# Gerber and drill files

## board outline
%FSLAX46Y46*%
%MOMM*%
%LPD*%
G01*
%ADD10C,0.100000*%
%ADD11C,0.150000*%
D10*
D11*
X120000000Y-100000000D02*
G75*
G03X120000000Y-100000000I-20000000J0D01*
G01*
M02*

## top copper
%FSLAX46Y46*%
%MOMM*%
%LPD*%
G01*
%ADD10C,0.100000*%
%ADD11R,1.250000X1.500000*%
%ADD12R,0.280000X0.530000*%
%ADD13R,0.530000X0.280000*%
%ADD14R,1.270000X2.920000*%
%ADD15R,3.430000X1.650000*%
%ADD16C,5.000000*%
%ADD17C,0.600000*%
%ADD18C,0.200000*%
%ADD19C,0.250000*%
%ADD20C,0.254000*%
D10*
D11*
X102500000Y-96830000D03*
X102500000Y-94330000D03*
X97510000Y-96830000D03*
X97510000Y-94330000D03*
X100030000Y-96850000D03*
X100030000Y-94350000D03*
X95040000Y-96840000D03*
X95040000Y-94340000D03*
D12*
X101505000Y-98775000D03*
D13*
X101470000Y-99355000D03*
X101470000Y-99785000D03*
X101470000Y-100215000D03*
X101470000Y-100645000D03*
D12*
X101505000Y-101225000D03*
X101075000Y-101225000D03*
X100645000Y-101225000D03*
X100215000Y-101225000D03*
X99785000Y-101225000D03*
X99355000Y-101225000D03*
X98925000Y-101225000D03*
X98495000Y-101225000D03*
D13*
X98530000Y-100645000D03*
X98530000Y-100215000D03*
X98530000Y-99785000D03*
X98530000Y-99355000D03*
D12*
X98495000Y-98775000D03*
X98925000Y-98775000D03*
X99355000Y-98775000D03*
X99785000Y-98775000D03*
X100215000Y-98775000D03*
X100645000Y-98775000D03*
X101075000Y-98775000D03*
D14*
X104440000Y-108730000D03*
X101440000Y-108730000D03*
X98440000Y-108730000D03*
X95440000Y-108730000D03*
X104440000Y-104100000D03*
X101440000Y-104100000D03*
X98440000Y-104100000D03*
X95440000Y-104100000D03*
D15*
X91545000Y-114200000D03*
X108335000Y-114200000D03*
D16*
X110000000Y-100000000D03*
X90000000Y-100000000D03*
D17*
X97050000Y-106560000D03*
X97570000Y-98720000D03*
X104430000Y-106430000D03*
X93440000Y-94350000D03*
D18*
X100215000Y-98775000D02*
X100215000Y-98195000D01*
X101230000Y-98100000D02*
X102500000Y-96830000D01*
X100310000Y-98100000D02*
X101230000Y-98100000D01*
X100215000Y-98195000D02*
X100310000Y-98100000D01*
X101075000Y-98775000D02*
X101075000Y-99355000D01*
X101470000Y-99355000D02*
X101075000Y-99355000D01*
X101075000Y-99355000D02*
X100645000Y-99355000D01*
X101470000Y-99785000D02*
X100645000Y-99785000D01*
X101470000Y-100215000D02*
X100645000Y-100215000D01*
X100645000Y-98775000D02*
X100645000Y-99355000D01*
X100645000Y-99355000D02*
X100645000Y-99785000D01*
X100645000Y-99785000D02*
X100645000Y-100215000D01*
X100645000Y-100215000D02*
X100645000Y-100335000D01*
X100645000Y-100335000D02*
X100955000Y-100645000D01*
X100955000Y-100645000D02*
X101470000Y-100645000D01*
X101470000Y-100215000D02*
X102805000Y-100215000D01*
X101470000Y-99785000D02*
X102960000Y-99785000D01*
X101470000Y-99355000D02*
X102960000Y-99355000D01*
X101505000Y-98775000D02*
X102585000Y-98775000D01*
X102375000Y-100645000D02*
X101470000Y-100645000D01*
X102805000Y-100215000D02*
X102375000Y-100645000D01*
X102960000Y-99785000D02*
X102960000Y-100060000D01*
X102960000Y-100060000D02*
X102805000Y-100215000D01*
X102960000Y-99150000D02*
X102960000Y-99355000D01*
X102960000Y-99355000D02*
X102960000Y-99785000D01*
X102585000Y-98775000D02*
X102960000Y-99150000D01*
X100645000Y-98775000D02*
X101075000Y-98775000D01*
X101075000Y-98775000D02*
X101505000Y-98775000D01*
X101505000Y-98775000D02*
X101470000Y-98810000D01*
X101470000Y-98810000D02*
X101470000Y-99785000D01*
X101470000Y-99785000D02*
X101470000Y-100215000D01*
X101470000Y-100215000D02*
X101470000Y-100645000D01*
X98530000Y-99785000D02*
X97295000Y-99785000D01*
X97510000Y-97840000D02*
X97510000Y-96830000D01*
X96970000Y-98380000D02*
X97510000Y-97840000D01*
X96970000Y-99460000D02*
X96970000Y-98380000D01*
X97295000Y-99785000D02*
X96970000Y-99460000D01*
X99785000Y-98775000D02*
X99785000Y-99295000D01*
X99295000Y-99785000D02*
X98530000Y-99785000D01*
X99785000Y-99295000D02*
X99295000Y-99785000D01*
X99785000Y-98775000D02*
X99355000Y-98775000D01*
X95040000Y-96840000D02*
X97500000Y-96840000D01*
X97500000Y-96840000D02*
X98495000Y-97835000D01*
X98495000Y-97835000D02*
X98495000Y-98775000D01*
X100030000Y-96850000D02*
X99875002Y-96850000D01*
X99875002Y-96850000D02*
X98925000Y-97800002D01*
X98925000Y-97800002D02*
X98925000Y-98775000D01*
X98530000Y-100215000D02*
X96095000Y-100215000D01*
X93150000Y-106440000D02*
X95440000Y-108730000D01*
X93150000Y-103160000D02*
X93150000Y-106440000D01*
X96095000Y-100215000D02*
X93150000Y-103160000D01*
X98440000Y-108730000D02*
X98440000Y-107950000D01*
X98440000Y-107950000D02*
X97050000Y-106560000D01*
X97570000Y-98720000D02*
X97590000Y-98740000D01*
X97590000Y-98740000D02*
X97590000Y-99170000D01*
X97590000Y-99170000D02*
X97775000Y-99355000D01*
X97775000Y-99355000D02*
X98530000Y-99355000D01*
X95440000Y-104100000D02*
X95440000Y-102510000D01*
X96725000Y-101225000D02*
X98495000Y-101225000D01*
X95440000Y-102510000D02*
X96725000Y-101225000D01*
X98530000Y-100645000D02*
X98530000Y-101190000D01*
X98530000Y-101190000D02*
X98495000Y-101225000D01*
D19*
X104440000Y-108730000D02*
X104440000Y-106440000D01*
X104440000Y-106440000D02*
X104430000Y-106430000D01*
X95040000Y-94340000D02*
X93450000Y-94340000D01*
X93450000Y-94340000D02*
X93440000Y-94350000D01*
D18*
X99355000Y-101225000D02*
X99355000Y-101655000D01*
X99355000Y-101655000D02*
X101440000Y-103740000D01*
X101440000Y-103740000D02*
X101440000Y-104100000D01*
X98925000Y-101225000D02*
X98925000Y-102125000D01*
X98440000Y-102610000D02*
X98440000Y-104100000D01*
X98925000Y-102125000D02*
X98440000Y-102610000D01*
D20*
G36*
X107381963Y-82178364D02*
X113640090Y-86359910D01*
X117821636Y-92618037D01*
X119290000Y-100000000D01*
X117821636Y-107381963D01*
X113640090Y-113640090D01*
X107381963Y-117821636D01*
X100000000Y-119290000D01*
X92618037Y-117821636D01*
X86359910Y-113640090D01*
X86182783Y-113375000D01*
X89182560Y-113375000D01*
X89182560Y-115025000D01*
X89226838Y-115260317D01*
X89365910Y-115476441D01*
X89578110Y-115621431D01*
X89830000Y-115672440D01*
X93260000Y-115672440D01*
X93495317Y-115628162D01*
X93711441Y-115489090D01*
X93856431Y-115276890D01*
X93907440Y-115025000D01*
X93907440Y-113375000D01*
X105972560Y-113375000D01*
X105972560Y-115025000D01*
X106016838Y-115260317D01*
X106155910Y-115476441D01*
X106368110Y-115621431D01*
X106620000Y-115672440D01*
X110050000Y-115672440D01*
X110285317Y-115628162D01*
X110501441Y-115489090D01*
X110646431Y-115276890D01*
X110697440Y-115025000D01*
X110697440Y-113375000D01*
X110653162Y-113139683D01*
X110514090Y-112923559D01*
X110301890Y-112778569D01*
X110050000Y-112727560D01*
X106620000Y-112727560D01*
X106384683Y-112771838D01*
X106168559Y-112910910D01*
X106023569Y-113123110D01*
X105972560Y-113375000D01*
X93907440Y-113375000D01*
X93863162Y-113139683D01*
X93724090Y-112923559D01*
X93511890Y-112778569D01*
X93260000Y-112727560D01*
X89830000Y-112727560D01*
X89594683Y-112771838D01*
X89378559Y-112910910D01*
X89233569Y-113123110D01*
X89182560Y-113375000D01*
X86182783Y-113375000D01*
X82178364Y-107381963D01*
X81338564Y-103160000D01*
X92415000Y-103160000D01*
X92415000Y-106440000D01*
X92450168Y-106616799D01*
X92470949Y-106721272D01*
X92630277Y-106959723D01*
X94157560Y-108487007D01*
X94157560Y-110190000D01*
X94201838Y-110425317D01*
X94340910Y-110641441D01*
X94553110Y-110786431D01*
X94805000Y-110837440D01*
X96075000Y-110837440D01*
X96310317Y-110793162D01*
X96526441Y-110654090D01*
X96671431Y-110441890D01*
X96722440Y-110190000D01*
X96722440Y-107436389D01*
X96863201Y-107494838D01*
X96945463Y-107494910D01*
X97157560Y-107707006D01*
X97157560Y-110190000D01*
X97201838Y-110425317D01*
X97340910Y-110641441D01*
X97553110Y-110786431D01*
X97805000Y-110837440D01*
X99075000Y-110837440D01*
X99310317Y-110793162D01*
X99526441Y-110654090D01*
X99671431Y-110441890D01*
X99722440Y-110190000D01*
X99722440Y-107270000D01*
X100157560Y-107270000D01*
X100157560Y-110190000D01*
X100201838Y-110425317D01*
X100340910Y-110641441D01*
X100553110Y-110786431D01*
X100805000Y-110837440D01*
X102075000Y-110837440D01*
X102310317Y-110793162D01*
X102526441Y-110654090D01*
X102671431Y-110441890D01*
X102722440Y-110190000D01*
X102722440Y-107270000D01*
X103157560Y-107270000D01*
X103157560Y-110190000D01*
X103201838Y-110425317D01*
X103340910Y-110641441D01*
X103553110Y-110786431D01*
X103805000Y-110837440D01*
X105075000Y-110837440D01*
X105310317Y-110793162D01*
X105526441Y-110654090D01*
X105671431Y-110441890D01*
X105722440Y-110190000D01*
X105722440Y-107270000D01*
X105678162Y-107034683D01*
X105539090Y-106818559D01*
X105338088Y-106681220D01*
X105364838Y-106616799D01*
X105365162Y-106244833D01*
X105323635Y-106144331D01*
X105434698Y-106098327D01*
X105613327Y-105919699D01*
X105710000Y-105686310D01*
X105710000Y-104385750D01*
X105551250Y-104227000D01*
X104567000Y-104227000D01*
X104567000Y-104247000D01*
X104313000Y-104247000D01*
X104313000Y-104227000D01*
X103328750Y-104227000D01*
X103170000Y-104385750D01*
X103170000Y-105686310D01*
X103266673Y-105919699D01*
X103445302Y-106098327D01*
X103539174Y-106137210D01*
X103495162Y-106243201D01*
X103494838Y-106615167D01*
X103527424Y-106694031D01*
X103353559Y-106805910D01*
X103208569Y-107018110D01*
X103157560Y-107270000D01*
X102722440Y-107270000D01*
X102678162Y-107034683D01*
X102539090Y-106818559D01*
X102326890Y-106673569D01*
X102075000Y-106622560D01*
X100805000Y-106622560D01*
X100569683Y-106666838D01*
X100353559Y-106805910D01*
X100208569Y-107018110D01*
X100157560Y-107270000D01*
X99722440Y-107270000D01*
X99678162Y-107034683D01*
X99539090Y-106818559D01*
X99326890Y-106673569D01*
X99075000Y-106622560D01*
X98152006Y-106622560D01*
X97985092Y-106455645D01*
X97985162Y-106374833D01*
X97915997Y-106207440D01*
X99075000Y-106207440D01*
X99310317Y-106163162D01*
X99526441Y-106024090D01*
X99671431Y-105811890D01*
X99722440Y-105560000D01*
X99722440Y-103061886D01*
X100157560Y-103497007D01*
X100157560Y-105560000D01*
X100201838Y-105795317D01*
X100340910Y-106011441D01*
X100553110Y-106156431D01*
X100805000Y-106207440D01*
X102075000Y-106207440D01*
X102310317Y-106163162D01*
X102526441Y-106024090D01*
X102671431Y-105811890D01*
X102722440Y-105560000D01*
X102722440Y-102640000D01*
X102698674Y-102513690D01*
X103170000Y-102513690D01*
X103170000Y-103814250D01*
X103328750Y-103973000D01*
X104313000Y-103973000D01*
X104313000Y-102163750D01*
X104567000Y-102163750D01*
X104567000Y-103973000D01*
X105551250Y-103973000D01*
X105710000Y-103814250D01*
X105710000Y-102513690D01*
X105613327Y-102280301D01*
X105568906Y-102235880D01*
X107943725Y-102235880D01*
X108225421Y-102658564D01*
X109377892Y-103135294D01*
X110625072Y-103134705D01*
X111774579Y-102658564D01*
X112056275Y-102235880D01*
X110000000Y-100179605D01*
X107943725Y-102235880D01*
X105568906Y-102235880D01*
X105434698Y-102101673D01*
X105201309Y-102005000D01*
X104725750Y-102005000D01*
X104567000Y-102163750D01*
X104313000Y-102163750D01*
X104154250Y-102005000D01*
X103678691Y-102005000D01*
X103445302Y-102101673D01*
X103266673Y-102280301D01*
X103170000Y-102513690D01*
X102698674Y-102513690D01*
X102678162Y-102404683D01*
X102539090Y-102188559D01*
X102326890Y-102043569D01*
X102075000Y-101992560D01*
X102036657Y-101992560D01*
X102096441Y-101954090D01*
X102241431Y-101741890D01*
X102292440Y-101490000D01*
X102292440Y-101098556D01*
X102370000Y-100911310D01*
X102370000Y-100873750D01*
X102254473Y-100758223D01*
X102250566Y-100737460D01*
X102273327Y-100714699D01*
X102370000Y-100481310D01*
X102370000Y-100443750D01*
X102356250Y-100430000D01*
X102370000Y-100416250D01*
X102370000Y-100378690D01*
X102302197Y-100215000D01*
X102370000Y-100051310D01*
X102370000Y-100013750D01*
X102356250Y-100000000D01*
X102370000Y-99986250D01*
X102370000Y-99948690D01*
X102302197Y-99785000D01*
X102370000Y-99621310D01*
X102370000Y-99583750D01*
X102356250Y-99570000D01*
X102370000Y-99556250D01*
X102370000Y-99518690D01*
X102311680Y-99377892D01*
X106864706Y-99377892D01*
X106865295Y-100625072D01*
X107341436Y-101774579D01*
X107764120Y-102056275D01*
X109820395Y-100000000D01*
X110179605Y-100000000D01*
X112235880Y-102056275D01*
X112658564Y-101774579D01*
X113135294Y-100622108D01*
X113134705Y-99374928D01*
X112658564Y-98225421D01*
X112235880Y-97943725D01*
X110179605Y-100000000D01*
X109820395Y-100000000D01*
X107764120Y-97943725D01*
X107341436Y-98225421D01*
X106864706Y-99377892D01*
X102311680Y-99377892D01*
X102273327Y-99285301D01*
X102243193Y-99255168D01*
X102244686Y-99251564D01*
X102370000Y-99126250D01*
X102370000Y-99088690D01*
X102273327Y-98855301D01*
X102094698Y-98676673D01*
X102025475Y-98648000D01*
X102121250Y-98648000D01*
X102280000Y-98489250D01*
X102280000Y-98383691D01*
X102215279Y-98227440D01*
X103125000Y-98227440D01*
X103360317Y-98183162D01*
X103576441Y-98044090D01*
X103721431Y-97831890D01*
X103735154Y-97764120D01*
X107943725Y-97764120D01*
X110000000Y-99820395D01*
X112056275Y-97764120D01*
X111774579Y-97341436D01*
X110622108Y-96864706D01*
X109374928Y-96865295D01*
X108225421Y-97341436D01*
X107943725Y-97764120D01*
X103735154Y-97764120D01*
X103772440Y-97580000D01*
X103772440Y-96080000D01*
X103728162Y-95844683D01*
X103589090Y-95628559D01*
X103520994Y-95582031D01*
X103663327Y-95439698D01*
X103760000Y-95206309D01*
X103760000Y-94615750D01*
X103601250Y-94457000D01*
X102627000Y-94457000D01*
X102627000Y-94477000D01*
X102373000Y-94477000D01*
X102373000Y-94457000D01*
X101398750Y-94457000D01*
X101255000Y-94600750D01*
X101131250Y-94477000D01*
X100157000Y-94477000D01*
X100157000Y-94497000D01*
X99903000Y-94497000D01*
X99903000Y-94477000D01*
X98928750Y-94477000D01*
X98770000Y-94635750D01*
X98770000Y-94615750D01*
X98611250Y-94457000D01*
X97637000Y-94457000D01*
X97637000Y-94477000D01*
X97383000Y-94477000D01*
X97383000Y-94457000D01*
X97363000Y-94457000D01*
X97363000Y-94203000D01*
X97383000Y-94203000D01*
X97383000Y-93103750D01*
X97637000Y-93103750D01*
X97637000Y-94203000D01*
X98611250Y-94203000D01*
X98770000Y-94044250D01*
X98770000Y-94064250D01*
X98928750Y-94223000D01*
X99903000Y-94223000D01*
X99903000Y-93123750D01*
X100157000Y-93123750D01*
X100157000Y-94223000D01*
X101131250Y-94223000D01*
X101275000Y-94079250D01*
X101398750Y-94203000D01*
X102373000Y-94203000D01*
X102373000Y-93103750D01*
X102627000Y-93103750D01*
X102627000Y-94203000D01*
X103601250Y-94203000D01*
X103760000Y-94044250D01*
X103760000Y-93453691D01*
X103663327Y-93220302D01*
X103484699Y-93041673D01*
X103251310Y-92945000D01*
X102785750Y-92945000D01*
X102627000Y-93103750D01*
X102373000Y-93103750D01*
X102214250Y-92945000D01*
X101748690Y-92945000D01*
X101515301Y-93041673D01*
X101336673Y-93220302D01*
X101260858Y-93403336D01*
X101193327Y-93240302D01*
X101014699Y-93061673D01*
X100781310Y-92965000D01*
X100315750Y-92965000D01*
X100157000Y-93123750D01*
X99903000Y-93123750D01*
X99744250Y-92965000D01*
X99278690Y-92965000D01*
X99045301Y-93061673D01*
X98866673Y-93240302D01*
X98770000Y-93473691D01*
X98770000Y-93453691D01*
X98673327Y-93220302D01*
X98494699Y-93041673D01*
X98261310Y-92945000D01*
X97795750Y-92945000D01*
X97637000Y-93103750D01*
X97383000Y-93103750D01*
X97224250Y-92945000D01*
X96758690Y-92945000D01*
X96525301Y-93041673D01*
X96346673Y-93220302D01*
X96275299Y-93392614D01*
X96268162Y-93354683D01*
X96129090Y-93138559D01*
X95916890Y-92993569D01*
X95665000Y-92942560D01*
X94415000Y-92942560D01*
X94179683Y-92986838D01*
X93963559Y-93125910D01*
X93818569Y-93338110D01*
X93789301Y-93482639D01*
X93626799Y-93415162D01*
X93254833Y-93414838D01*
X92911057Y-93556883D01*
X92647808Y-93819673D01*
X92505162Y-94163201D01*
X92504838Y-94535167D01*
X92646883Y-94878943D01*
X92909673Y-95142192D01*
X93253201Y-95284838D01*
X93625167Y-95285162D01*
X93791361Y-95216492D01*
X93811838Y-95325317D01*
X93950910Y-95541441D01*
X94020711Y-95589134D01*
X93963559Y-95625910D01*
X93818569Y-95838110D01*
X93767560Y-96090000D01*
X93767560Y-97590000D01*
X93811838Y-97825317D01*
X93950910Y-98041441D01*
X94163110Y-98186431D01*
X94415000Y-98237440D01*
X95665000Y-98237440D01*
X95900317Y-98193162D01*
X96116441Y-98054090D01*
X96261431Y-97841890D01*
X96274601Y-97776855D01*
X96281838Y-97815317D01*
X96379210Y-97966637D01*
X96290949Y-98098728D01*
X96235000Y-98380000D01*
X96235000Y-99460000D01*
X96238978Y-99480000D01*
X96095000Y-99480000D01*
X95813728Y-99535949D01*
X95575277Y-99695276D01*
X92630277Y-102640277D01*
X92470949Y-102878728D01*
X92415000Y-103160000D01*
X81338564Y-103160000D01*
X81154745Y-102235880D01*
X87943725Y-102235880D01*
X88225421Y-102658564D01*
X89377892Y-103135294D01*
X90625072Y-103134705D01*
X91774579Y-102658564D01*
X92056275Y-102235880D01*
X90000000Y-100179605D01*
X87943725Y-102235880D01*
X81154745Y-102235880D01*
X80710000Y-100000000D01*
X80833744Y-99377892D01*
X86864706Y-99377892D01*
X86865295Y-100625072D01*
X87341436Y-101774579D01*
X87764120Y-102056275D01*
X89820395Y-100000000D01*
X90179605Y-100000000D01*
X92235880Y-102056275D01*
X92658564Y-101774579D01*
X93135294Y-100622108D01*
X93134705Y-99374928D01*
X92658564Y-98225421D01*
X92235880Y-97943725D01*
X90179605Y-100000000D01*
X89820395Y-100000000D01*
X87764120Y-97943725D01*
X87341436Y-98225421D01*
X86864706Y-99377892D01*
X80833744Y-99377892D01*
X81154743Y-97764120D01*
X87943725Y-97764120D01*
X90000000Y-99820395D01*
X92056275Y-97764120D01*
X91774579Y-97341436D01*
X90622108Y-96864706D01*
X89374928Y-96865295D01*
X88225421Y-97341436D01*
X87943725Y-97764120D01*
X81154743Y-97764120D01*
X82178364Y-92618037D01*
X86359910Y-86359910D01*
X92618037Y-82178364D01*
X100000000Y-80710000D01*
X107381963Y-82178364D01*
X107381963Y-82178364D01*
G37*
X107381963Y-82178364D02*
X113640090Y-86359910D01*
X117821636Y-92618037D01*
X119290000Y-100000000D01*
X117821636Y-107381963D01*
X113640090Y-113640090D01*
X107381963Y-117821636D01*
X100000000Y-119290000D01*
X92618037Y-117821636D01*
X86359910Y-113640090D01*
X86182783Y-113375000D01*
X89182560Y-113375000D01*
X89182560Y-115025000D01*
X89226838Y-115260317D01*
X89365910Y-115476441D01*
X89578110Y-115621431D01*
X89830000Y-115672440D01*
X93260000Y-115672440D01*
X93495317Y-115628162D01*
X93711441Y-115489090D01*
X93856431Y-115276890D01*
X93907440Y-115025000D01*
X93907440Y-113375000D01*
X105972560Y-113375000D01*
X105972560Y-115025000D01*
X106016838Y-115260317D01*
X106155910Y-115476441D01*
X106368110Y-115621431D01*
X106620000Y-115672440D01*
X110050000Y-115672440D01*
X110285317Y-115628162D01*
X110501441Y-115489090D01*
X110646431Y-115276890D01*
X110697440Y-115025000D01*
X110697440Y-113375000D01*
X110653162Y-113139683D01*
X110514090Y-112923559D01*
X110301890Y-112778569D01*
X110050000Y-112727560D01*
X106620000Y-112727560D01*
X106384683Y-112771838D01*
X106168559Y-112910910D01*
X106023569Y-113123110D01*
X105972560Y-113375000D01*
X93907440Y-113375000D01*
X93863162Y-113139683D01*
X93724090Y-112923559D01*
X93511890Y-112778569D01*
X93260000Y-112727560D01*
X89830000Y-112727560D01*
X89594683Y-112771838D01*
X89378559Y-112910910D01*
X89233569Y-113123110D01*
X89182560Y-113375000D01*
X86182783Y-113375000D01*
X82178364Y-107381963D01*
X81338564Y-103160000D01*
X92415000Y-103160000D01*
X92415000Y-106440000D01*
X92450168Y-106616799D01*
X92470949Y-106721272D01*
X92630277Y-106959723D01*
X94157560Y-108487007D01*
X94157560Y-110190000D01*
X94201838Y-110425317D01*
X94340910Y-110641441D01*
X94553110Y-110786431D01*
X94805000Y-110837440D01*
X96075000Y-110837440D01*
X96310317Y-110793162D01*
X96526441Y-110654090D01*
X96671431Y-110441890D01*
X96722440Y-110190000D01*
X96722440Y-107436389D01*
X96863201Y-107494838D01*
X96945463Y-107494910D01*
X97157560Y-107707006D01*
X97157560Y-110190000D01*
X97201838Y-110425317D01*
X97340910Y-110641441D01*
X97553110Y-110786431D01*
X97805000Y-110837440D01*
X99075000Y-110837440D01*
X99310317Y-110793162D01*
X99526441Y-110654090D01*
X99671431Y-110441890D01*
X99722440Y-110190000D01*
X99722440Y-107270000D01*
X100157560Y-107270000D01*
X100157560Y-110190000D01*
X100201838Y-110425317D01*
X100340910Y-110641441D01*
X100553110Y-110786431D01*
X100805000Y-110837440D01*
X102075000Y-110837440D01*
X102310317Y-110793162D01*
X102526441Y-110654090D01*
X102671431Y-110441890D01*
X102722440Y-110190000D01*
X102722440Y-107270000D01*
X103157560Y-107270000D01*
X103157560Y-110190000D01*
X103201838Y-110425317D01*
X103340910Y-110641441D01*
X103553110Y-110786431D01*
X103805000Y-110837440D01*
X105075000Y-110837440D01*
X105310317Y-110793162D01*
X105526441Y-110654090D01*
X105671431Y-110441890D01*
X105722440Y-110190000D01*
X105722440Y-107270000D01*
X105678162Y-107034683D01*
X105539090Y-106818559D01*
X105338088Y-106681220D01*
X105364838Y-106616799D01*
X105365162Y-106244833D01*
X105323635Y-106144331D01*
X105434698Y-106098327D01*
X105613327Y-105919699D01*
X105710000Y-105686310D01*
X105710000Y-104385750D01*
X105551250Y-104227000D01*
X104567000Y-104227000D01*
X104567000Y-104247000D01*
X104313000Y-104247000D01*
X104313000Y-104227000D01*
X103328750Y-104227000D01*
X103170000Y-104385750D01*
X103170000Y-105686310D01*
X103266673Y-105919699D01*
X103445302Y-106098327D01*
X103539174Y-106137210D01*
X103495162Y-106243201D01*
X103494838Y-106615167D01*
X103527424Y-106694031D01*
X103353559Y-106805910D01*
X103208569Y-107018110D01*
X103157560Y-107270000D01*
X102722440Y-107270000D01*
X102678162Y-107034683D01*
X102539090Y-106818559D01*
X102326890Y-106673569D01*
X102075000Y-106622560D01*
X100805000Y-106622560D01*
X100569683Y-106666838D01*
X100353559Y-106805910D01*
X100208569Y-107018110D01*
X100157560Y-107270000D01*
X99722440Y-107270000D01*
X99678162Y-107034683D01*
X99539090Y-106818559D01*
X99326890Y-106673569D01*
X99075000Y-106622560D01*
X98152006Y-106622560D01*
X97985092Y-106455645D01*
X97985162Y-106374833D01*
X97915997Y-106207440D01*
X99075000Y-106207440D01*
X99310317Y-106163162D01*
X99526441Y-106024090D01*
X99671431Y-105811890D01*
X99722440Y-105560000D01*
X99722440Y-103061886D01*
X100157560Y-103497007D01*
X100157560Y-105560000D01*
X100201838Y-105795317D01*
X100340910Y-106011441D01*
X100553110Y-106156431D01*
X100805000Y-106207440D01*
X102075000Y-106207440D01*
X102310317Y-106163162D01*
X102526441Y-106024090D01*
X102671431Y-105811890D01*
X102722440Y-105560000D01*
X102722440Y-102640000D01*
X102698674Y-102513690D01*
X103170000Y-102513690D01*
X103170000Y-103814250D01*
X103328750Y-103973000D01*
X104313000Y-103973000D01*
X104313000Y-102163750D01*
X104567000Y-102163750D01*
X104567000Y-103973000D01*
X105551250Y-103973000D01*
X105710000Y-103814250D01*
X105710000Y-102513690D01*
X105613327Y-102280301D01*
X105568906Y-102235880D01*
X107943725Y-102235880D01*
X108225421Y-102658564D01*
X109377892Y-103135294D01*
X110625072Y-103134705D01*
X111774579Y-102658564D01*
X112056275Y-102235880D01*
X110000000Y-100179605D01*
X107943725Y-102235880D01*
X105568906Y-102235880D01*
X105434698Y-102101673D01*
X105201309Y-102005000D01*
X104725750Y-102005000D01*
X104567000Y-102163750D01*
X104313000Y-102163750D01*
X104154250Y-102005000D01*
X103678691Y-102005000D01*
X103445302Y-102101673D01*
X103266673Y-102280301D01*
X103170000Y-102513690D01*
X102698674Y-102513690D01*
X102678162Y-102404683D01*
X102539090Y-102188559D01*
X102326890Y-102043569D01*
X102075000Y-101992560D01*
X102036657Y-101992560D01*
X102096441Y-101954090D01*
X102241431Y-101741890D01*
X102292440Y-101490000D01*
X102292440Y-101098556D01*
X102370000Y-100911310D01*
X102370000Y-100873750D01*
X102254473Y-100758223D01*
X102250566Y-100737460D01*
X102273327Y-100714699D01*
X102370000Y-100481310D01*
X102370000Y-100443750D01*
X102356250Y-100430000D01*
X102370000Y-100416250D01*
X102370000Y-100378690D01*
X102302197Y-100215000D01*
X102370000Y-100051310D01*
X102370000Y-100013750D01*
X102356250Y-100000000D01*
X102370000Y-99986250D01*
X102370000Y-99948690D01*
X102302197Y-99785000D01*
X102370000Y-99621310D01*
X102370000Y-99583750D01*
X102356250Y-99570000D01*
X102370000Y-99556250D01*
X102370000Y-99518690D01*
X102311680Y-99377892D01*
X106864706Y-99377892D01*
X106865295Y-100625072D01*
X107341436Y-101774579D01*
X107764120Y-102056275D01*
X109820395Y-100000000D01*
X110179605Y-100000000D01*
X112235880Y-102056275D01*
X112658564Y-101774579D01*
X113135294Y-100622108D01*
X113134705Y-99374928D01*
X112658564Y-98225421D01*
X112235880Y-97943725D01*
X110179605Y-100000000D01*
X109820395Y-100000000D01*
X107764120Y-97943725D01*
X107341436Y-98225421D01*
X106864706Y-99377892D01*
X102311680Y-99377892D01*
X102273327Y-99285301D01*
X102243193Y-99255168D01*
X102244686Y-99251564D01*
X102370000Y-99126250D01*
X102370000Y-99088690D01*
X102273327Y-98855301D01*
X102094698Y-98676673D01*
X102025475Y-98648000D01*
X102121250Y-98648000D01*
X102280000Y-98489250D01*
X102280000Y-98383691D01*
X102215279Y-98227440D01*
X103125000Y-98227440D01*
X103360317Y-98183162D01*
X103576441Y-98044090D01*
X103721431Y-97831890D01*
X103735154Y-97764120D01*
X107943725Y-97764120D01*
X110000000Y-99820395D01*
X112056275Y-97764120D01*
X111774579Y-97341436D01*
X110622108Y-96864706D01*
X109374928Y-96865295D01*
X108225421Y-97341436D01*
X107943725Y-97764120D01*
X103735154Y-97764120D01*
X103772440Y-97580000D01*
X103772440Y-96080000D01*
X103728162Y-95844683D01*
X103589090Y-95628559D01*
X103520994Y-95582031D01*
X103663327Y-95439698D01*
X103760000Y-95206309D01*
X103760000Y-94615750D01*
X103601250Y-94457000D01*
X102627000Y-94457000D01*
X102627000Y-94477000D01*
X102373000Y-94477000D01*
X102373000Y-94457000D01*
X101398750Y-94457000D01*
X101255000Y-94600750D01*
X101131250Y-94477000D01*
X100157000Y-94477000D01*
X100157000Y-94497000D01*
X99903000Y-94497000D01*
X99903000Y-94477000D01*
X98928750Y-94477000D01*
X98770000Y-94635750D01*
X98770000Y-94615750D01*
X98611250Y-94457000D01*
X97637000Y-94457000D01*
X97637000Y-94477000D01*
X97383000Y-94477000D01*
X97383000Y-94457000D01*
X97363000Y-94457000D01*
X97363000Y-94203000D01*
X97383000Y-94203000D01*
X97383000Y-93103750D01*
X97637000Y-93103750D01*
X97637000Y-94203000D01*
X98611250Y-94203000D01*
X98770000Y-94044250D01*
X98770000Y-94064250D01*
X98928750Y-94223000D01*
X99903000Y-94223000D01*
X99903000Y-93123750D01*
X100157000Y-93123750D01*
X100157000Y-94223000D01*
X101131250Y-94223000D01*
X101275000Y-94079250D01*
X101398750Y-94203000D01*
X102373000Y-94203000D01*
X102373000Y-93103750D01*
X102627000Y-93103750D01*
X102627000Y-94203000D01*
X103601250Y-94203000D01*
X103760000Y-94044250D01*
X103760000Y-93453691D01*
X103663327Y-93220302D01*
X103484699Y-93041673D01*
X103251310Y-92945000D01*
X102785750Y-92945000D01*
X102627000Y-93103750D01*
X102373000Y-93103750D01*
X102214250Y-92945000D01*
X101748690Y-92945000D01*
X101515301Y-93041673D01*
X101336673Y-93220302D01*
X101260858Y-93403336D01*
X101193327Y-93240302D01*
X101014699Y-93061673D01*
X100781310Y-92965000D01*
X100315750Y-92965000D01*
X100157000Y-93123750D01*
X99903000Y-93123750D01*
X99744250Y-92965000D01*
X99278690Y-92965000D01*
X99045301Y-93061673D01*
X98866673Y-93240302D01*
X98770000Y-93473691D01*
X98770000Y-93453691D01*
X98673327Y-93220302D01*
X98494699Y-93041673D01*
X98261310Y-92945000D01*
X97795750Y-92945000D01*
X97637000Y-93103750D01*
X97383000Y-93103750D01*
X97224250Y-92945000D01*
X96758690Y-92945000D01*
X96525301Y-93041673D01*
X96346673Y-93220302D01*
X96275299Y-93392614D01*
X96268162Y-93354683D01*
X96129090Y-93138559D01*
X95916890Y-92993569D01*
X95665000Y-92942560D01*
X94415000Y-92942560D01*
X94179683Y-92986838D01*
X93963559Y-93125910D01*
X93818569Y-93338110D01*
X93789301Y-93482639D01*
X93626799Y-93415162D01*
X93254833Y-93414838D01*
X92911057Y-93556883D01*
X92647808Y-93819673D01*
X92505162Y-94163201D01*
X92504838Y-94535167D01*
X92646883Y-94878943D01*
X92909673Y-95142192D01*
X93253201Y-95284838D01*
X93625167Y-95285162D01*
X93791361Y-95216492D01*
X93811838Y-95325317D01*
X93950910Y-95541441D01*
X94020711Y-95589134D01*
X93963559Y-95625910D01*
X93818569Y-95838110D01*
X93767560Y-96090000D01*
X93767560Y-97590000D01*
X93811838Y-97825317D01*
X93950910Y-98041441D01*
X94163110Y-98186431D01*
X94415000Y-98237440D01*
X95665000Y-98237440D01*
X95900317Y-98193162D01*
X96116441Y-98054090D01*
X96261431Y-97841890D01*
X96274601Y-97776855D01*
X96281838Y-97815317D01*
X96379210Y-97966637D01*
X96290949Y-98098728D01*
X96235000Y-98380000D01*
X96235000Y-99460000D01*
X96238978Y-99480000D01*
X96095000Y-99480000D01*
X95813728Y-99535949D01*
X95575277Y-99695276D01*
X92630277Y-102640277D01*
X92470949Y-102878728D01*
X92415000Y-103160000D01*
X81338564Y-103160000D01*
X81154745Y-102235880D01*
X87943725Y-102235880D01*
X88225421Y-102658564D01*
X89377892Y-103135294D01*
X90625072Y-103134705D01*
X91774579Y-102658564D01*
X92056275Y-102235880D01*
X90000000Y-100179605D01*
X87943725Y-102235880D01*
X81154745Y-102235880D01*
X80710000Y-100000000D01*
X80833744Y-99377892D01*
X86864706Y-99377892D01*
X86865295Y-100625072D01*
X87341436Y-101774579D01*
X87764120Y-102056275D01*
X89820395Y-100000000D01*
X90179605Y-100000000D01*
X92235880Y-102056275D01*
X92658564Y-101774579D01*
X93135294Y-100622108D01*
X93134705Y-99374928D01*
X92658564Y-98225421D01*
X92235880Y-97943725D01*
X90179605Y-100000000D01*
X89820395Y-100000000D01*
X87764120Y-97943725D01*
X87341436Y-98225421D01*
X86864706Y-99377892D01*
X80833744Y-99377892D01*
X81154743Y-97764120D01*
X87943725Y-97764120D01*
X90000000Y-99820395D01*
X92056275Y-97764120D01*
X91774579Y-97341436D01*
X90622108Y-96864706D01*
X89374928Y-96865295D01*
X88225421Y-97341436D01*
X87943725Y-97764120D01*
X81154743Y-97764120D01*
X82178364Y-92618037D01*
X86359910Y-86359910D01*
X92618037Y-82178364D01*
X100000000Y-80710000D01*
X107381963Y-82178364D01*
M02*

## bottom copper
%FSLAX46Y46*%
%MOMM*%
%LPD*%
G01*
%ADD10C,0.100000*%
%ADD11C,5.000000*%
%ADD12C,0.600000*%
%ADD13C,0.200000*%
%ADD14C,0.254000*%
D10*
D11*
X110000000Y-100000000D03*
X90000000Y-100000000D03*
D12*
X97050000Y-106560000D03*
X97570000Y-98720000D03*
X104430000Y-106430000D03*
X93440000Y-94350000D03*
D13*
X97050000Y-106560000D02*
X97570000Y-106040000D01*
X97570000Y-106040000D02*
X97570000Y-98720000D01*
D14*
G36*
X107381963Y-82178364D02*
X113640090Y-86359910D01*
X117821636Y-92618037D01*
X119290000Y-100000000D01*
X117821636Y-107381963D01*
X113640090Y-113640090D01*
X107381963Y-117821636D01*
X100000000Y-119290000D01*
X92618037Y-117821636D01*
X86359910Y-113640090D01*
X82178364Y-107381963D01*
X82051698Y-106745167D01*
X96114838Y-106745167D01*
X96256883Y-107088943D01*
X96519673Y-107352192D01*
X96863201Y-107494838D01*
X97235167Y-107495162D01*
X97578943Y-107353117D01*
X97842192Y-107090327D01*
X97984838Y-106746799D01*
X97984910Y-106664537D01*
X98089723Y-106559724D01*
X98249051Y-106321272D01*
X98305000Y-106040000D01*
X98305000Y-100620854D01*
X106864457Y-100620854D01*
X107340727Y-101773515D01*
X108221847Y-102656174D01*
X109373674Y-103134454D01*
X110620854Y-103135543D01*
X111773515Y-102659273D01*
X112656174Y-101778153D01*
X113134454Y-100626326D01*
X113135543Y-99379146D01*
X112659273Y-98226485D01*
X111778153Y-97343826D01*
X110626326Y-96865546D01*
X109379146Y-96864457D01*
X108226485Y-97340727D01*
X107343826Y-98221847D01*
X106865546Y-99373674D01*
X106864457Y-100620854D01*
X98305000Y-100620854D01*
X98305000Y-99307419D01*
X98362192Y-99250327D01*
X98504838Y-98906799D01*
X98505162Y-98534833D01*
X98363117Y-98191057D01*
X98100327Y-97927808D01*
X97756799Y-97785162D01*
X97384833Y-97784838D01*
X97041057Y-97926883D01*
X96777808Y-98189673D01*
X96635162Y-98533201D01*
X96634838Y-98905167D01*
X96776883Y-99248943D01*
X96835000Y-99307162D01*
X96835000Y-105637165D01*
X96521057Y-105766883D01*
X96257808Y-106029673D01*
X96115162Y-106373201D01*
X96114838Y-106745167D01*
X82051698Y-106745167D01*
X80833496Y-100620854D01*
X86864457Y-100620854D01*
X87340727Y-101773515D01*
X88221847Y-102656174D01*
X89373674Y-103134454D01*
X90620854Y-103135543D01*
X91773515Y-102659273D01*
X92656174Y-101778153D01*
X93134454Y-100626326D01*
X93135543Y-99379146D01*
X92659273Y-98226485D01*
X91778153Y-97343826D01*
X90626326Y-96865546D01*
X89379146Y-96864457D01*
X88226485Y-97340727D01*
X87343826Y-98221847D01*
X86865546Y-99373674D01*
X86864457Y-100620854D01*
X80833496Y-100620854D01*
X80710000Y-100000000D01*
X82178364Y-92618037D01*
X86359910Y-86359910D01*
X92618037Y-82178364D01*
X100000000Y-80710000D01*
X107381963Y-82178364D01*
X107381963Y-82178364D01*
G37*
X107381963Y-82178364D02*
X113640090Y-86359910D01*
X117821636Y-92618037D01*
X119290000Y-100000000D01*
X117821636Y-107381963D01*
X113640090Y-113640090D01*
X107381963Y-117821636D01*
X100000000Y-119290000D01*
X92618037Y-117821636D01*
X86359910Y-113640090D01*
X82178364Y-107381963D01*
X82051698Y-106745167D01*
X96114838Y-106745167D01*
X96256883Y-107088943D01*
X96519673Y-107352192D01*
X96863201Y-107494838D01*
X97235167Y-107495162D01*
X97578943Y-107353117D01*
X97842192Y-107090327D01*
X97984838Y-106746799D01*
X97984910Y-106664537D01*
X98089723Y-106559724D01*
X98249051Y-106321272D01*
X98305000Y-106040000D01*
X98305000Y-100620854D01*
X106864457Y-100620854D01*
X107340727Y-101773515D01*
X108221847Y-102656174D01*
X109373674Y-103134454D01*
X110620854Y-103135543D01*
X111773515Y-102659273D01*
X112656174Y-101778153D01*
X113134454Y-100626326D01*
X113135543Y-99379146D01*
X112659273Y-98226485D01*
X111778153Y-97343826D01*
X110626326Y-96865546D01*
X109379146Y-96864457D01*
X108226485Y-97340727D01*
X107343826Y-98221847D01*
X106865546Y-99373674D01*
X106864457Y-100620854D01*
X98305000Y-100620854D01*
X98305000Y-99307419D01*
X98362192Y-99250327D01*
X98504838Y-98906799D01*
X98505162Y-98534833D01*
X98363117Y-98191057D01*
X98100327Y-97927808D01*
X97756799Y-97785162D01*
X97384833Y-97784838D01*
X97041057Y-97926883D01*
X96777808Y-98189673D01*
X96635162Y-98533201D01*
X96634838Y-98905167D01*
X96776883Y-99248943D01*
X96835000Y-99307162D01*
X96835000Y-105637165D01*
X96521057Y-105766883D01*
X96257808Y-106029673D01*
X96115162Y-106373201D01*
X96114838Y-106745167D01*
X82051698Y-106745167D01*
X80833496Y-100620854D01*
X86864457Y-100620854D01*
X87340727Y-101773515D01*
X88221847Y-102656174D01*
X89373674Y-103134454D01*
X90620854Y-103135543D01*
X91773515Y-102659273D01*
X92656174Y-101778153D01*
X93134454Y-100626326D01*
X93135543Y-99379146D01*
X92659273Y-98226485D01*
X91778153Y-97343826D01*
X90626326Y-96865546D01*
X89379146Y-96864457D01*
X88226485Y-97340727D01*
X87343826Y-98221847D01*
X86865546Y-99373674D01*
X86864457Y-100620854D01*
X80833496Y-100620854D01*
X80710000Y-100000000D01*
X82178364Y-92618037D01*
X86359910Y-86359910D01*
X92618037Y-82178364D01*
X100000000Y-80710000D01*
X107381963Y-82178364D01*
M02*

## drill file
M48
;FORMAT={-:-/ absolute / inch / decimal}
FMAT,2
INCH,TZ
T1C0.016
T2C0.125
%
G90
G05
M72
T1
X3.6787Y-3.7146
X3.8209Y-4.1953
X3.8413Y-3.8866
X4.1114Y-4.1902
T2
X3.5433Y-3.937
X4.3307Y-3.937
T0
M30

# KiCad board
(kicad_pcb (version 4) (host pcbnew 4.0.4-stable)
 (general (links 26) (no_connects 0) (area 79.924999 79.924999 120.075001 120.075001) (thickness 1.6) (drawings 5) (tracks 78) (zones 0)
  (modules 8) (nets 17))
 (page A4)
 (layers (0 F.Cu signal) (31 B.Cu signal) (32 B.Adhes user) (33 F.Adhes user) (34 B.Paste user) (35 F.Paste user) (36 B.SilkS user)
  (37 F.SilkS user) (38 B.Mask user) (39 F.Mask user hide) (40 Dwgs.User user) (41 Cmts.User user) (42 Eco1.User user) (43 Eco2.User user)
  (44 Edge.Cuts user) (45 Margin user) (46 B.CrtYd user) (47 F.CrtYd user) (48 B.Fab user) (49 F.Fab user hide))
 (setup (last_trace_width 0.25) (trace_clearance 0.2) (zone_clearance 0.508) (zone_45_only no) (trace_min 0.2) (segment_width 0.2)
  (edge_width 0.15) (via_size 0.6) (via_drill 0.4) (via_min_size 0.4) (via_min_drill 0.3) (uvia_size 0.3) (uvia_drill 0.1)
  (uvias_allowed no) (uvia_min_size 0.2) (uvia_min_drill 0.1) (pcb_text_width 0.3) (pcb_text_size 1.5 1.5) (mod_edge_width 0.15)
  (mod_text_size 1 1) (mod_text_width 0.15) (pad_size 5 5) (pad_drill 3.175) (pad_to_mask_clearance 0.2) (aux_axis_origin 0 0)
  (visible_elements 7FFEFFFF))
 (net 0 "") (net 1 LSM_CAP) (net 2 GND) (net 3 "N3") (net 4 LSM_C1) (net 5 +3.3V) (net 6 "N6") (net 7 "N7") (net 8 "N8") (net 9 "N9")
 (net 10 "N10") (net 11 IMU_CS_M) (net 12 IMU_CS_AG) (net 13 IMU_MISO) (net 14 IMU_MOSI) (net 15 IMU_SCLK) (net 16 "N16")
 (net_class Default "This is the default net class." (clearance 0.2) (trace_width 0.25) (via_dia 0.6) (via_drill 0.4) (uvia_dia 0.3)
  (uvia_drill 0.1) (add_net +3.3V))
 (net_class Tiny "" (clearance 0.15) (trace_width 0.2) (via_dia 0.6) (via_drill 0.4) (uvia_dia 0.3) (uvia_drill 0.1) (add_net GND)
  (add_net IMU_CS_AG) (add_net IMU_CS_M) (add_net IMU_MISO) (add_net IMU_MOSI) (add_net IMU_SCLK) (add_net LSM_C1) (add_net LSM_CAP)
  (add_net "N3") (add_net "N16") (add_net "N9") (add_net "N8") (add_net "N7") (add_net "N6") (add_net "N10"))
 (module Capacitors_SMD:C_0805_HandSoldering (layer F.Cu) (at 102.5 95.58 90)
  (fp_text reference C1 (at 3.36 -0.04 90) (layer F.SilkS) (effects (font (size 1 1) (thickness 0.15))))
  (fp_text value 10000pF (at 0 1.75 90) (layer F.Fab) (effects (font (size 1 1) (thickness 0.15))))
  (pad 1 smd rect (at -1.25 0 90) (size 1.5 1.25) (layers F.Cu F.Paste F.Mask) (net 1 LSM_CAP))
  (pad 2 smd rect (at 1.25 0 90) (size 1.5 1.25) (layers F.Cu F.Paste F.Mask) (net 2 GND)))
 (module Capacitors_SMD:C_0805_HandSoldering (layer F.Cu) (at 97.51 95.58 90)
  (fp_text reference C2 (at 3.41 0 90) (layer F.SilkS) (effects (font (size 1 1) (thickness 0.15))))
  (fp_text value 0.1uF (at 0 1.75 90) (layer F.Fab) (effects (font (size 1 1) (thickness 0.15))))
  (pad 1 smd rect (at -1.25 0 90) (size 1.5 1.25) (layers F.Cu F.Paste F.Mask) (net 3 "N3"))
  (pad 2 smd rect (at 1.25 0 90) (size 1.5 1.25) (layers F.Cu F.Paste F.Mask) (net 2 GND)))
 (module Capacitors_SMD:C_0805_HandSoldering (layer F.Cu) (at 100.03 95.6 90)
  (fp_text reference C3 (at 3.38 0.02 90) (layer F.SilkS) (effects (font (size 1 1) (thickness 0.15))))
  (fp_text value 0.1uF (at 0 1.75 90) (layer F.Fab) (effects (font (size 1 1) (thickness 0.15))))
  (pad 1 smd rect (at -1.25 0 90) (size 1.5 1.25) (layers F.Cu F.Paste F.Mask) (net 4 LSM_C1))
  (pad 2 smd rect (at 1.25 0 90) (size 1.5 1.25) (layers F.Cu F.Paste F.Mask) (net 2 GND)))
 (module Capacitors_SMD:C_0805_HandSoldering (layer F.Cu) (at 95.04 95.59 90)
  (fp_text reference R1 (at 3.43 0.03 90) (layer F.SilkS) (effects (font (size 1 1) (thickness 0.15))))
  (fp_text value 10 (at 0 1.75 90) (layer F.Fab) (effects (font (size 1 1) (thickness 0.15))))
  (pad 1 smd rect (at -1.25 0 90) (size 1.5 1.25) (layers F.Cu F.Paste F.Mask) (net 3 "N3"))
  (pad 2 smd rect (at 1.25 0 90) (size 1.5 1.25) (layers F.Cu F.Paste F.Mask) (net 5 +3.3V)))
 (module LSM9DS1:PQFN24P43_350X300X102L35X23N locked (layer F.Cu) (at 100 100)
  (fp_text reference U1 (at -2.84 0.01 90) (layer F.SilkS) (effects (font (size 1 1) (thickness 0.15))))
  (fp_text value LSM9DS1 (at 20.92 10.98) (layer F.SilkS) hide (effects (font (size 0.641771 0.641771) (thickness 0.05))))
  (pad 18 smd rect (at 1.505 -1.225 270) (size 0.53 0.28) (layers F.Cu F.Paste F.Mask) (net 2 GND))
  (pad 17 smd rect (at 1.47 -0.645) (size 0.53 0.28) (layers F.Cu F.Paste F.Mask) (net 2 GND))
  (pad 16 smd rect (at 1.47 -0.215) (size 0.53 0.28) (layers F.Cu F.Paste F.Mask) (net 2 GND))
  (pad 15 smd rect (at 1.47 0.215) (size 0.53 0.28) (layers F.Cu F.Paste F.Mask) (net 2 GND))
  (pad 14 smd rect (at 1.47 0.645) (size 0.53 0.28) (layers F.Cu F.Paste F.Mask) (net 2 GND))
  (pad 13 smd rect (at 1.505 1.225 90) (size 0.53 0.28) (layers F.Cu F.Paste F.Mask) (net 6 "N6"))
  (pad 12 smd rect (at 1.075 1.225 270) (size 0.53 0.28) (layers F.Cu F.Paste F.Mask) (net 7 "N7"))
  (pad 11 smd rect (at 0.645 1.225 90) (size 0.53 0.28) (layers F.Cu F.Paste F.Mask) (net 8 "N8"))
  (pad 10 smd rect (at 0.215 1.225 270) (size 0.53 0.28) (layers F.Cu F.Paste F.Mask) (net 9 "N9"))
  (pad 9 smd rect (at -0.215 1.225 90) (size 0.53 0.28) (layers F.Cu F.Paste F.Mask) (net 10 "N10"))
  (pad 8 smd rect (at -0.645 1.225 90) (size 0.53 0.28) (layers F.Cu F.Paste F.Mask) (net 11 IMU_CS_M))
  (pad 7 smd rect (at -1.075 1.225 90) (size 0.53 0.28) (layers F.Cu F.Paste F.Mask) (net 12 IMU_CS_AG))
  (pad 6 smd rect (at -1.505 1.225 270) (size 0.53 0.28) (layers F.Cu F.Paste F.Mask) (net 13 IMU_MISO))
  (pad 5 smd rect (at -1.47 0.645 180) (size 0.53 0.28) (layers F.Cu F.Paste F.Mask) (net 13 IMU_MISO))
  (pad 4 smd rect (at -1.47 0.215 180) (size 0.53 0.28) (layers F.Cu F.Paste F.Mask) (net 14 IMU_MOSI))
  (pad 3 smd rect (at -1.47 -0.215 180) (size 0.53 0.28) (layers F.Cu F.Paste F.Mask) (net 3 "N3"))
  (pad 2 smd rect (at -1.47 -0.645 180) (size 0.53 0.28) (layers F.Cu F.Paste F.Mask) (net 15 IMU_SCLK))
  (pad 1 smd rect (at -1.505 -1.225 270) (size 0.53 0.28) (layers F.Cu F.Paste F.Mask) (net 3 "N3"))
  (pad 24 smd rect (at -1.075 -1.225 270) (size 0.53 0.28) (layers F.Cu F.Paste F.Mask) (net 4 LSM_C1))
  (pad 23 smd rect (at -0.645 -1.225 270) (size 0.53 0.28) (layers F.Cu F.Paste F.Mask) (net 3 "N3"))
  (pad 22 smd rect (at -0.215 -1.225 270) (size 0.53 0.28) (layers F.Cu F.Paste F.Mask) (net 3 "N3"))
  (pad 21 smd rect (at 0.215 -1.225 270) (size 0.53 0.28) (layers F.Cu F.Paste F.Mask) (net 1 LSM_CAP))
  (pad 20 smd rect (at 0.645 -1.225 270) (size 0.53 0.28) (layers F.Cu F.Paste F.Mask) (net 2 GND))
  (pad 19 smd rect (at 1.075 -1.225 270) (size 0.53 0.28) (layers F.Cu F.Paste F.Mask) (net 2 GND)))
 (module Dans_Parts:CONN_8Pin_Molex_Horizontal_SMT (layer F.Cu) (at 104.44 108.73)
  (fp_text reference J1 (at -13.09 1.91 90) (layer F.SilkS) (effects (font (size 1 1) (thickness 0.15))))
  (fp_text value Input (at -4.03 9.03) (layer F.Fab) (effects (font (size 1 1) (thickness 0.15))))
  (pad 1 smd rect (at 0 0) (size 1.27 2.92) (layers F.Cu F.Paste F.Mask) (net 5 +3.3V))
  (pad 2 smd rect (at -3 0) (size 1.27 2.92) (layers F.Cu F.Paste F.Mask) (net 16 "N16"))
  (pad 3 smd rect (at -6 0) (size 1.27 2.92) (layers F.Cu F.Paste F.Mask) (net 15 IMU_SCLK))
  (pad 4 smd rect (at -9 0) (size 1.27 2.92) (layers F.Cu F.Paste F.Mask) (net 14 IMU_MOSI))
  (pad 5 smd rect (at 0 -4.63) (size 1.27 2.92) (layers F.Cu F.Paste F.Mask) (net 2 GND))
  (pad 6 smd rect (at -3 -4.63) (size 1.27 2.92) (layers F.Cu F.Paste F.Mask) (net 11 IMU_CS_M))
  (pad 7 smd rect (at -6 -4.63) (size 1.27 2.92) (layers F.Cu F.Paste F.Mask) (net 12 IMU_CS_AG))
  (pad 8 smd rect (at -9 -4.63) (size 1.27 2.92) (layers F.Cu F.Paste F.Mask) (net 13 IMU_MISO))
  (pad "" smd rect (at -12.895 5.47) (size 3.43 1.65) (layers F.Cu F.Paste F.Mask))
  (pad "" smd rect (at 3.895 5.47) (size 3.43 1.65) (layers F.Cu F.Paste F.Mask)))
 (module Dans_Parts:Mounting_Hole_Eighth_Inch (layer F.Cu) (at 111.93 99.75)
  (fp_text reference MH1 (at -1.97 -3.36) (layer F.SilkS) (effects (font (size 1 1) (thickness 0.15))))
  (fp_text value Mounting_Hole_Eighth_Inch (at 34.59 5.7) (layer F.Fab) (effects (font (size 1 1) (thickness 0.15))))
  (pad 1 thru_hole circle (at -1.93 0.25) (size 5 5) (drill 3.175) (layers *.Cu *.Mask) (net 2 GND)))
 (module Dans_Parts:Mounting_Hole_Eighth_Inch (layer F.Cu) (at 87.21 99.48)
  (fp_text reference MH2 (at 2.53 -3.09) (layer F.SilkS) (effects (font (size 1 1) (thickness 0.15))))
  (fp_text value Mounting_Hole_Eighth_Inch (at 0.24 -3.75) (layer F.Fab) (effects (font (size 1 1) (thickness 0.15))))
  (pad 1 thru_hole circle (at 2.79 0.52) (size 5 5) (drill 3.175) (layers *.Cu *.Mask) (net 2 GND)))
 (gr_circle (center 100 100) (end 120 100) (layer Edge.Cuts) (width 0.15))
 (segment (start 100.215 98.775) (end 100.215 98.195) (width 0.2) (layer F.Cu) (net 1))
 (segment (start 101.23 98.1) (end 102.5 96.83) (width 0.2) (layer F.Cu) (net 1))
 (segment (start 100.31 98.1) (end 101.23 98.1) (width 0.2) (layer F.Cu) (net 1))
 (segment (start 100.215 98.195) (end 100.31 98.1) (width 0.2) (layer F.Cu) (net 1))
 (segment (start 101.075 98.775) (end 101.075 99.355) (width 0.2) (layer F.Cu) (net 2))
 (segment (start 101.47 99.355) (end 101.075 99.355) (width 0.2) (layer F.Cu) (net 2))
 (segment (start 101.075 99.355) (end 100.645 99.355) (width 0.2) (layer F.Cu) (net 2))
 (segment (start 101.47 99.785) (end 100.645 99.785) (width 0.2) (layer F.Cu) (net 2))
 (segment (start 101.47 100.215) (end 100.645 100.215) (width 0.2) (layer F.Cu) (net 2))
 (segment (start 100.645 98.775) (end 100.645 99.355) (width 0.2) (layer F.Cu) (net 2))
 (segment (start 100.645 99.355) (end 100.645 99.785) (width 0.2) (layer F.Cu) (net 2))
 (segment (start 100.645 99.785) (end 100.645 100.215) (width 0.2) (layer F.Cu) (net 2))
 (segment (start 100.645 100.215) (end 100.645 100.335) (width 0.2) (layer F.Cu) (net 2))
 (segment (start 100.645 100.335) (end 100.955 100.645) (width 0.2) (layer F.Cu) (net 2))
 (segment (start 100.955 100.645) (end 101.47 100.645) (width 0.2) (layer F.Cu) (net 2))
 (segment (start 101.47 100.215) (end 102.805 100.215) (width 0.2) (layer F.Cu) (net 2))
 (segment (start 101.47 99.785) (end 102.96 99.785) (width 0.2) (layer F.Cu) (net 2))
 (segment (start 101.47 99.355) (end 102.96 99.355) (width 0.2) (layer F.Cu) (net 2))
 (segment (start 101.505 98.775) (end 102.585 98.775) (width 0.2) (layer F.Cu) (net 2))
 (segment (start 102.375 100.645) (end 101.47 100.645) (width 0.2) (layer F.Cu) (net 2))
 (segment (start 102.805 100.215) (end 102.375 100.645) (width 0.2) (layer F.Cu) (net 2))
 (segment (start 102.96 99.785) (end 102.96 100.06) (width 0.2) (layer F.Cu) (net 2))
 (segment (start 102.96 100.06) (end 102.805 100.215) (width 0.2) (layer F.Cu) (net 2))
 (segment (start 102.96 99.15) (end 102.96 99.355) (width 0.2) (layer F.Cu) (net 2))
 (segment (start 102.96 99.355) (end 102.96 99.785) (width 0.2) (layer F.Cu) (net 2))
 (segment (start 102.585 98.775) (end 102.96 99.15) (width 0.2) (layer F.Cu) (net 2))
 (segment (start 100.645 98.775) (end 101.075 98.775) (width 0.2) (layer F.Cu) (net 2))
 (segment (start 101.075 98.775) (end 101.505 98.775) (width 0.2) (layer F.Cu) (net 2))
 (segment (start 101.505 98.775) (end 101.47 98.81) (width 0.2) (layer F.Cu) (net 2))
 (segment (start 101.47 98.81) (end 101.47 99.785) (width 0.2) (layer F.Cu) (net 2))
 (segment (start 101.47 99.785) (end 101.47 100.215) (width 0.2) (layer F.Cu) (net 2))
 (segment (start 101.47 100.215) (end 101.47 100.645) (width 0.2) (layer F.Cu) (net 2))
 (segment (start 98.53 99.785) (end 97.295 99.785) (width 0.2) (layer F.Cu) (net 3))
 (segment (start 97.51 97.84) (end 97.51 96.83) (width 0.2) (layer F.Cu) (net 3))
 (segment (start 96.97 98.38) (end 97.51 97.84) (width 0.2) (layer F.Cu) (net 3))
 (segment (start 96.97 99.46) (end 96.97 98.38) (width 0.2) (layer F.Cu) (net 3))
 (segment (start 97.295 99.785) (end 96.97 99.46) (width 0.2) (layer F.Cu) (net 3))
 (segment (start 99.785 98.775) (end 99.785 99.295) (width 0.2) (layer F.Cu) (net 3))
 (segment (start 99.295 99.785) (end 98.53 99.785) (width 0.2) (layer F.Cu) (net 3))
 (segment (start 99.785 99.295) (end 99.295 99.785) (width 0.2) (layer F.Cu) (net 3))
 (segment (start 99.785 98.775) (end 99.355 98.775) (width 0.2) (layer F.Cu) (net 3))
 (segment (start 95.04 96.84) (end 97.5 96.84) (width 0.2) (layer F.Cu) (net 3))
 (segment (start 97.5 96.84) (end 98.495 97.835) (width 0.2) (layer F.Cu) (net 3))
 (segment (start 98.495 97.835) (end 98.495 98.775) (width 0.2) (layer F.Cu) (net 3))
 (segment (start 100.03 96.85) (end 99.875002 96.85) (width 0.2) (layer F.Cu) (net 4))
 (segment (start 99.875002 96.85) (end 98.925 97.800002) (width 0.2) (layer F.Cu) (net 4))
 (segment (start 98.925 97.800002) (end 98.925 98.775) (width 0.2) (layer F.Cu) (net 4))
 (segment (start 98.53 100.215) (end 96.095 100.215) (width 0.2) (layer F.Cu) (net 14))
 (segment (start 93.15 106.44) (end 95.44 108.73) (width 0.2) (layer F.Cu) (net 14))
 (segment (start 93.15 103.16) (end 93.15 106.44) (width 0.2) (layer F.Cu) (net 14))
 (segment (start 96.095 100.215) (end 93.15 103.16) (width 0.2) (layer F.Cu) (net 14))
 (segment (start 98.44 108.73) (end 98.44 107.95) (width 0.2) (layer F.Cu) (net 15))
 (segment (start 98.44 107.95) (end 97.05 106.56) (width 0.2) (layer F.Cu) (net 15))
 (via (at 97.05 106.56) (size 0.6) (drill 0.4) (layers F.Cu B.Cu) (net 15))
 (segment (start 97.05 106.56) (end 97.57 106.04) (width 0.2) (layer B.Cu) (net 15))
 (segment (start 97.57 106.04) (end 97.57 98.72) (width 0.2) (layer B.Cu) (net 15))
 (via (at 97.57 98.72) (size 0.6) (drill 0.4) (layers F.Cu B.Cu) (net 15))
 (segment (start 97.57 98.72) (end 97.59 98.74) (width 0.2) (layer F.Cu) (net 15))
 (segment (start 97.59 98.74) (end 97.59 99.17) (width 0.2) (layer F.Cu) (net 15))
 (segment (start 97.59 99.17) (end 97.775 99.355) (width 0.2) (layer F.Cu) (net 15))
 (segment (start 97.775 99.355) (end 98.53 99.355) (width 0.2) (layer F.Cu) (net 15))
 (segment (start 95.44 104.1) (end 95.44 102.51) (width 0.2) (layer F.Cu) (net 13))
 (segment (start 96.725 101.225) (end 98.495 101.225) (width 0.2) (layer F.Cu) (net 13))
 (segment (start 95.44 102.51) (end 96.725 101.225) (width 0.2) (layer F.Cu) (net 13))
 (segment (start 98.53 100.645) (end 98.53 101.19) (width 0.2) (layer F.Cu) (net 13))
 (segment (start 98.53 101.19) (end 98.495 101.225) (width 0.2) (layer F.Cu) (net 13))
 (segment (start 104.44 108.73) (end 104.44 106.44) (width 0.25) (layer F.Cu) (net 5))
 (via (at 104.43 106.43) (size 0.6) (drill 0.4) (layers F.Cu B.Cu) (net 5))
 (segment (start 104.44 106.44) (end 104.43 106.43) (width 0.25) (layer F.Cu) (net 5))
 (segment (start 95.04 94.34) (end 93.45 94.34) (width 0.25) (layer F.Cu) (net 5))
 (via (at 93.44 94.35) (size 0.6) (drill 0.4) (layers F.Cu B.Cu) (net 5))
 (segment (start 93.45 94.34) (end 93.44 94.35) (width 0.25) (layer F.Cu) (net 5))
 (segment (start 99.355 101.225) (end 99.355 101.655) (width 0.2) (layer F.Cu) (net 11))
 (segment (start 99.355 101.655) (end 101.44 103.74) (width 0.2) (layer F.Cu) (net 11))
 (segment (start 101.44 103.74) (end 101.44 104.1) (width 0.2) (layer F.Cu) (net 11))
 (segment (start 98.925 101.225) (end 98.925 102.125) (width 0.2) (layer F.Cu) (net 12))
 (segment (start 98.44 102.61) (end 98.44 104.1) (width 0.2) (layer F.Cu) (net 12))
 (segment (start 98.925 102.125) (end 98.44 102.61) (width 0.2) (layer F.Cu) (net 12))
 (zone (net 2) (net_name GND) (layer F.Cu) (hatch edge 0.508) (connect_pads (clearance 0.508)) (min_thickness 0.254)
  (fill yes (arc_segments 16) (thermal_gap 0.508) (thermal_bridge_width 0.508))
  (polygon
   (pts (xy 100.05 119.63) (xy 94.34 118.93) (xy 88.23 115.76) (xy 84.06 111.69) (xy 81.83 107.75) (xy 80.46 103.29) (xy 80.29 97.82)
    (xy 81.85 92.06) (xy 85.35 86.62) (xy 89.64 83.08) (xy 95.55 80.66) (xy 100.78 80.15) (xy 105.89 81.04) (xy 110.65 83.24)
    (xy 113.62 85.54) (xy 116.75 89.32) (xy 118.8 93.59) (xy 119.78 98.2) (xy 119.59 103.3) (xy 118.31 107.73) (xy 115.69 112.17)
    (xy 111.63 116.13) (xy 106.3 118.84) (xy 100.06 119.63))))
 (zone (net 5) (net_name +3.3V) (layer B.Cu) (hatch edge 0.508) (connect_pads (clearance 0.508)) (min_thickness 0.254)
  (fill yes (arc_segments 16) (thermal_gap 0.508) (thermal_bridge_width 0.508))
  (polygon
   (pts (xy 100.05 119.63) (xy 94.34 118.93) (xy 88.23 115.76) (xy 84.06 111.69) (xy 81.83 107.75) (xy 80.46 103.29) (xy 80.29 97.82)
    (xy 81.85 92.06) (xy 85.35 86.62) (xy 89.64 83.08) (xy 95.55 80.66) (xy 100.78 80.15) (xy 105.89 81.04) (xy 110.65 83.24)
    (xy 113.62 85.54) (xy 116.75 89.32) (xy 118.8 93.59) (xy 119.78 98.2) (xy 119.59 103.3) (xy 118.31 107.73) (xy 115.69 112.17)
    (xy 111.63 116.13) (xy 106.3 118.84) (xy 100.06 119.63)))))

